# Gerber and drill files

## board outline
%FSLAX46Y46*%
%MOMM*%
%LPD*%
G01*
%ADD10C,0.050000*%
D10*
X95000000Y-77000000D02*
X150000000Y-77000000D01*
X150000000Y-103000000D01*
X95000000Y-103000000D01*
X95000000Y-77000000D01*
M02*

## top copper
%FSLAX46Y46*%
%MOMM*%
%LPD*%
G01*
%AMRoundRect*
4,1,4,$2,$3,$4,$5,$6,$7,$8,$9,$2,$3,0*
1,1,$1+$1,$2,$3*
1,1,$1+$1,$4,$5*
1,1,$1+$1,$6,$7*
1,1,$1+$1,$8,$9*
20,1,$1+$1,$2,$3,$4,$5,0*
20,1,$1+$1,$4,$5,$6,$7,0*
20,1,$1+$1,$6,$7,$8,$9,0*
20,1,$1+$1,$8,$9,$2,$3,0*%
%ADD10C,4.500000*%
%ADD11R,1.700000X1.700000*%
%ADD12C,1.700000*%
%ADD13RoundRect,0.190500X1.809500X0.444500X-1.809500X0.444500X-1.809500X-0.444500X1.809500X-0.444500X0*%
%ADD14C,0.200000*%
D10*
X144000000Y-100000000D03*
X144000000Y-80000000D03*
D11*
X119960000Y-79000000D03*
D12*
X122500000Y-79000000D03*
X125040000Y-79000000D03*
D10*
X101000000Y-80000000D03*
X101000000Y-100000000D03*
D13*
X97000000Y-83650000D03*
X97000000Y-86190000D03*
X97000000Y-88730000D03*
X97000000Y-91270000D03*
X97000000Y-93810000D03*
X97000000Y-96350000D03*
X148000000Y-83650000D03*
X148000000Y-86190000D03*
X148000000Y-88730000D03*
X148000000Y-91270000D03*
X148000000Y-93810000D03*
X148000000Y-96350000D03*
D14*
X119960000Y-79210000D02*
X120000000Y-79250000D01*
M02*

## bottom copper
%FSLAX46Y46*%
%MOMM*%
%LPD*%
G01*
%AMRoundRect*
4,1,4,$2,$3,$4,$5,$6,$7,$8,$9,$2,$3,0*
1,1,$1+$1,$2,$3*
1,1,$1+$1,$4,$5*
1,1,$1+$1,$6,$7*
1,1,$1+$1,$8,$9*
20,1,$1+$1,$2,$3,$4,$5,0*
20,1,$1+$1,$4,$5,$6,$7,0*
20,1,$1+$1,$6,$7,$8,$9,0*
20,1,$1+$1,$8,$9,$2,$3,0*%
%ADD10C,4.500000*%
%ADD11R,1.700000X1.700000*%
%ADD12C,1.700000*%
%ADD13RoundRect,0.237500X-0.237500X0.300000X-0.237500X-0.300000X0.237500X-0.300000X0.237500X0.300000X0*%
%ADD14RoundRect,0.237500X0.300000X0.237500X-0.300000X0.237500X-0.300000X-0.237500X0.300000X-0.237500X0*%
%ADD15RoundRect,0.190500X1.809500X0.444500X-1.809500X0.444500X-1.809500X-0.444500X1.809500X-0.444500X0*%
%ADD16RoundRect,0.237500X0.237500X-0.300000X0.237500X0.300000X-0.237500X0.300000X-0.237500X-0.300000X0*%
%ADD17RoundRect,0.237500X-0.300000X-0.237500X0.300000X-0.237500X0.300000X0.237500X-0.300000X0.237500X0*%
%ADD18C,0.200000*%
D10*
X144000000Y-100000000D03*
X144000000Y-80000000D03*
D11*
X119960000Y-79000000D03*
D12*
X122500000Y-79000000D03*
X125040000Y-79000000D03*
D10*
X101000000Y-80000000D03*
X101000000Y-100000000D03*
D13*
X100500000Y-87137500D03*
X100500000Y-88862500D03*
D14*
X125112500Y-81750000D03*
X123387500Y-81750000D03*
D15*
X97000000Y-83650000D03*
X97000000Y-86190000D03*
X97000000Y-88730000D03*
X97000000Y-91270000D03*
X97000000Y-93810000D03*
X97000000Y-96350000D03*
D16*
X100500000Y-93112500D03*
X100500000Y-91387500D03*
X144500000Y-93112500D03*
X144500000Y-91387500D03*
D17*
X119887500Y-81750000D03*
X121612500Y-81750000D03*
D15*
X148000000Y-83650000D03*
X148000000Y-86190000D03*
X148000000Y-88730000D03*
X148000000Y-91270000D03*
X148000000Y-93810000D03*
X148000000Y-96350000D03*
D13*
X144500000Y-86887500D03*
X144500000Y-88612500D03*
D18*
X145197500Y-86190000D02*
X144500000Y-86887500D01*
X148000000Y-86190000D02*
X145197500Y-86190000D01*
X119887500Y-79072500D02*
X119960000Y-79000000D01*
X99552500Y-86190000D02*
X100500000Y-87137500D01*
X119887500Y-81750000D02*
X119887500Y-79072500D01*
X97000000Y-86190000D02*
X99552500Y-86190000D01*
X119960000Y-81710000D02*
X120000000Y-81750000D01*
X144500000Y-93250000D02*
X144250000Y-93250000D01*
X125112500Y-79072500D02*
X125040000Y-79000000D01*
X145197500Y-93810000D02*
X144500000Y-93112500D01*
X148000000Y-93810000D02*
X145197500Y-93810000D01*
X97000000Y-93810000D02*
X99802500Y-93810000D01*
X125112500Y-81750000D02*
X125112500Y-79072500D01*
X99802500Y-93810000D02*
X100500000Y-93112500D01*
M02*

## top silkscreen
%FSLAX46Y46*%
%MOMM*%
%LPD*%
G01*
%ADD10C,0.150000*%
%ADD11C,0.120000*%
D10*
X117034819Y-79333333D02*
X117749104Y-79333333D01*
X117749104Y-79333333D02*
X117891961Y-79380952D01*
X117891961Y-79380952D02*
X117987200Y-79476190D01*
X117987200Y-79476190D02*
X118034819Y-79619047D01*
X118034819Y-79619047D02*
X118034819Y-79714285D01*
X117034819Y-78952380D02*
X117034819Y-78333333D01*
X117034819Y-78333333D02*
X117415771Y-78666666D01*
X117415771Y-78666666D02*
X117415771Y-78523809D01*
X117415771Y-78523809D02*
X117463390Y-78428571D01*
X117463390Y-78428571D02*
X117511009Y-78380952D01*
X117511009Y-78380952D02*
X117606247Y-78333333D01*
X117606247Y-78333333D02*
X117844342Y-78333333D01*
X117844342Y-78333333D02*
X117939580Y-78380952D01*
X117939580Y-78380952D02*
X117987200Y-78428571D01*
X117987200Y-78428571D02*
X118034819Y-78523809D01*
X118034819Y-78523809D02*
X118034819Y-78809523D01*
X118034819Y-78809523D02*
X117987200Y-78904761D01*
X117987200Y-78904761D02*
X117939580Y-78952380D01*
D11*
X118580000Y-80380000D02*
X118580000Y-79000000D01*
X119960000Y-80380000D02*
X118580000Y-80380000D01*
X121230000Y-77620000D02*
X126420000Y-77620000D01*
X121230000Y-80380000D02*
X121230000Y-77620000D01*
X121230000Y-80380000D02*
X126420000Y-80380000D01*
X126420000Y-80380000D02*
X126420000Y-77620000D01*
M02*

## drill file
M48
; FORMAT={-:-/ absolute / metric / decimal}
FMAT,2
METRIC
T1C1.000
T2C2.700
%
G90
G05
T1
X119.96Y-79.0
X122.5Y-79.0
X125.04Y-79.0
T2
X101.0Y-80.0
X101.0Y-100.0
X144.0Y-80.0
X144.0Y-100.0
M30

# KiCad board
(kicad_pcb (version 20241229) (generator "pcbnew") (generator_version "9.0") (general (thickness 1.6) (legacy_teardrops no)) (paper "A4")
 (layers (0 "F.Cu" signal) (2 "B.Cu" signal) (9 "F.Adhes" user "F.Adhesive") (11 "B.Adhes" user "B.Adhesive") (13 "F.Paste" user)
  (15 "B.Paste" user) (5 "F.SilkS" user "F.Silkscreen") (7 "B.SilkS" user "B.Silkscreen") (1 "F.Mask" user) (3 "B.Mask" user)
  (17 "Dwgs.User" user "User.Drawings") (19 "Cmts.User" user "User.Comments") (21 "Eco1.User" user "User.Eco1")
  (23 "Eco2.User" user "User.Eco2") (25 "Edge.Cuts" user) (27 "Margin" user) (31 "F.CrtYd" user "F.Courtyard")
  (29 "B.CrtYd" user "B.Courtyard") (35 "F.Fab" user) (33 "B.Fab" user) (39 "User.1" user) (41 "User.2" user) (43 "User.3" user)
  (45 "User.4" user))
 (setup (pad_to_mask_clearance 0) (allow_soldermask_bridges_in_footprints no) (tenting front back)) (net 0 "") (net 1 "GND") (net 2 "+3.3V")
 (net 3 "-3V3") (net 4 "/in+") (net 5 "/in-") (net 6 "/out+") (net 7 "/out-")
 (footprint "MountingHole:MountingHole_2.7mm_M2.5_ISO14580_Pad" (layer "F.Cu") (at 144 100)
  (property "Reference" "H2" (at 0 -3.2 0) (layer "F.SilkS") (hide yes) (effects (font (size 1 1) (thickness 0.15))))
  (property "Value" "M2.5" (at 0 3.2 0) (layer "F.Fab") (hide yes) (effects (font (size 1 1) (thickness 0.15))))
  (pad "1" thru_hole circle (at 0 0) (size 4.5 4.5) (drill 2.7) (layers "*.Cu" "*.Mask") (remove_unused_layers no) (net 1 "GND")
   (zone_connect 2)))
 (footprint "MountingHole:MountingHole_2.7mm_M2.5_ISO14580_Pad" (layer "F.Cu") (at 144 80)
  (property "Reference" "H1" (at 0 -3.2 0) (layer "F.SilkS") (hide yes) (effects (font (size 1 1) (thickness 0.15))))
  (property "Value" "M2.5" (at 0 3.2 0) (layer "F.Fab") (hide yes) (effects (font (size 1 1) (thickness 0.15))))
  (pad "1" thru_hole circle (at 0 0) (size 4.5 4.5) (drill 2.7) (layers "*.Cu" "*.Mask") (remove_unused_layers no) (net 1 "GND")
   (zone_connect 2)))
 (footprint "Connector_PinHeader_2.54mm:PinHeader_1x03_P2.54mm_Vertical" (layer "F.Cu") (at 119.96 79 90)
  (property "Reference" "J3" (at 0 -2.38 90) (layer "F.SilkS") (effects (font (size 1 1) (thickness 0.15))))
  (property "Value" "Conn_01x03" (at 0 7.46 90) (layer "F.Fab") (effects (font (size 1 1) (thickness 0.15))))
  (fp_line (start -1.38 -1.38) (end 0 -1.38) (stroke (width 0.12) (type solid)) (layer "F.SilkS"))
  (fp_line (start -1.38 0) (end -1.38 -1.38) (stroke (width 0.12) (type solid)) (layer "F.SilkS"))
  (fp_line (start 1.38 1.27) (end 1.38 6.46) (stroke (width 0.12) (type solid)) (layer "F.SilkS"))
  (fp_line (start -1.38 1.27) (end 1.38 1.27) (stroke (width 0.12) (type solid)) (layer "F.SilkS"))
  (fp_line (start -1.38 1.27) (end -1.38 6.46) (stroke (width 0.12) (type solid)) (layer "F.SilkS"))
  (fp_line (start -1.38 6.46) (end 1.38 6.46) (stroke (width 0.12) (type solid)) (layer "F.SilkS"))
  (pad "1" thru_hole rect (at 0 0 90) (size 1.7 1.7) (drill 1) (layers "*.Cu" "*.Mask") (remove_unused_layers no) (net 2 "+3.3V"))
  (pad "2" thru_hole circle (at 0 2.54 90) (size 1.7 1.7) (drill 1) (layers "*.Cu" "*.Mask") (remove_unused_layers no) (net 1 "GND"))
  (pad "3" thru_hole circle (at 0 5.08 90) (size 1.7 1.7) (drill 1) (layers "*.Cu" "*.Mask") (remove_unused_layers no) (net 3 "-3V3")))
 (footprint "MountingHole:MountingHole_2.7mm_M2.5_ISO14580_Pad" (layer "F.Cu") (at 101 80)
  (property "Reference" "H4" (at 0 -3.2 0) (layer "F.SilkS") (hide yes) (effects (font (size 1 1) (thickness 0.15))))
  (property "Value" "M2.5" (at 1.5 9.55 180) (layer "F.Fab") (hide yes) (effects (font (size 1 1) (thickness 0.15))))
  (pad "1" thru_hole circle (at 0 0) (size 4.5 4.5) (drill 2.7) (layers "*.Cu" "*.Mask") (remove_unused_layers no) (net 1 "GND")
   (zone_connect 2)))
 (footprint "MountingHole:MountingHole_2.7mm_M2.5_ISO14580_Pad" (layer "F.Cu") (at 101 100)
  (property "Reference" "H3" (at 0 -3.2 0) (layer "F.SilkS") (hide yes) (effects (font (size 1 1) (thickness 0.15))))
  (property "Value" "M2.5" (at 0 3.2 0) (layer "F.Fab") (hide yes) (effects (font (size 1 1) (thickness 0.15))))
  (pad "1" thru_hole circle (at 0 0) (size 4.5 4.5) (drill 2.7) (layers "*.Cu" "*.Mask") (remove_unused_layers no) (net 1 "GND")
   (zone_connect 2)))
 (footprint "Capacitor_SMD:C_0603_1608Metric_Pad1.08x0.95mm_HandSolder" (layer "B.Cu") (at 100.5 88 -90)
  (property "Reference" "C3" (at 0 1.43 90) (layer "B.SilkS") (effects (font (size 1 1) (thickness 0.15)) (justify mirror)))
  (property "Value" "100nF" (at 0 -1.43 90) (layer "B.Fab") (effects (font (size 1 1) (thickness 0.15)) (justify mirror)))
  (pad "1" smd roundrect (at -0.8625 0 270) (size 1.075 0.95) (layers "B.Cu" "B.Mask" "B.Paste") (roundrect_rratio 0.25) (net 2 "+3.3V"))
  (pad "2" smd roundrect (at 0.8625 0 270) (size 1.075 0.95) (layers "B.Cu" "B.Mask" "B.Paste") (roundrect_rratio 0.25) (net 1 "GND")))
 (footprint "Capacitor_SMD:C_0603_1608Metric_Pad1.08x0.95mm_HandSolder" (layer "B.Cu") (at 124.25 81.75 180)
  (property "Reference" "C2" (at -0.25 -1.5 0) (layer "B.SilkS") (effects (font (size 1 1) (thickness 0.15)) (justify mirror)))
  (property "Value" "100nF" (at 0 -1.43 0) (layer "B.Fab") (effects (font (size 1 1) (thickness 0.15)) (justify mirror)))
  (pad "1" smd roundrect (at -0.8625 0 180) (size 1.075 0.95) (layers "B.Cu" "B.Mask" "B.Paste") (roundrect_rratio 0.25) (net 3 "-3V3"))
  (pad "2" smd roundrect (at 0.8625 0 180) (size 1.075 0.95) (layers "B.Cu" "B.Mask" "B.Paste") (roundrect_rratio 0.25) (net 1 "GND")))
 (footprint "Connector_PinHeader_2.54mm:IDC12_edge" (layer "B.Cu") (at 97 83.65 180)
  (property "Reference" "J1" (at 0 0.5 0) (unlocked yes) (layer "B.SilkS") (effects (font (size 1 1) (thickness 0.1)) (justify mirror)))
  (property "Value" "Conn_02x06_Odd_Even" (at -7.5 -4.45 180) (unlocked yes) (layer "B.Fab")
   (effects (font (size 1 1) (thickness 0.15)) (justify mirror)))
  (pad "1" smd roundrect (at 0 0 180) (size 4 1.27) (layers "B.Cu" "B.Mask" "B.Paste") (roundrect_rratio 0.15) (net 1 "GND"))
  (pad "2" smd roundrect (at 0 0 180) (size 4 1.27) (layers "F.Cu" "F.Mask" "F.Paste") (roundrect_rratio 0.15) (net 1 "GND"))
  (pad "3" smd roundrect (at 0 -2.54 180) (size 4 1.27) (layers "B.Cu" "B.Mask" "B.Paste") (roundrect_rratio 0.15) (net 2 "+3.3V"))
  (pad "4" smd roundrect (at 0 -2.54 180) (size 4 1.27) (layers "F.Cu" "F.Mask" "F.Paste") (roundrect_rratio 0.15) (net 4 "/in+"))
  (pad "5" smd roundrect (at 0 -5.08 180) (size 4 1.27) (layers "B.Cu" "B.Mask" "B.Paste") (roundrect_rratio 0.15) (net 1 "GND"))
  (pad "6" smd roundrect (at 0 -5.08 180) (size 4 1.27) (layers "F.Cu" "F.Mask" "F.Paste") (roundrect_rratio 0.15) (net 1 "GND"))
  (pad "7" smd roundrect (at 0 -7.62 180) (size 4 1.27) (layers "B.Cu" "B.Mask" "B.Paste") (roundrect_rratio 0.15) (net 1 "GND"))
  (pad "8" smd roundrect (at 0 -7.62 180) (size 4 1.27) (layers "F.Cu" "F.Mask" "F.Paste") (roundrect_rratio 0.15) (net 1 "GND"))
  (pad "9" smd roundrect (at 0 -10.16 180) (size 4 1.27) (layers "B.Cu" "B.Mask" "B.Paste") (roundrect_rratio 0.15) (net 3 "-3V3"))
  (pad "10" smd roundrect (at 0 -10.16 180) (size 4 1.27) (layers "F.Cu" "F.Mask" "F.Paste") (roundrect_rratio 0.15) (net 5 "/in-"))
  (pad "11" smd roundrect (at 0 -12.7 180) (size 4 1.27) (layers "B.Cu" "B.Mask" "B.Paste") (roundrect_rratio 0.15) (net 1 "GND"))
  (pad "12" smd roundrect (at 0 -12.7 180) (size 4 1.27) (layers "F.Cu" "F.Mask" "F.Paste") (roundrect_rratio 0.15) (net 1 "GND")))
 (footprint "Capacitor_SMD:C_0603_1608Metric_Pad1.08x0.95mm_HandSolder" (layer "B.Cu") (at 100.5 92.25 90)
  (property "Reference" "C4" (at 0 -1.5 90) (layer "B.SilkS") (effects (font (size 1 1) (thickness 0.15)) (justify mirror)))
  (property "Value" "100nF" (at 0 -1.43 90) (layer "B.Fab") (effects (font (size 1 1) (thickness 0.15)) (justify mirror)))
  (pad "1" smd roundrect (at -0.8625 0 90) (size 1.075 0.95) (layers "B.Cu" "B.Mask" "B.Paste") (roundrect_rratio 0.25) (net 3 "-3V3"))
  (pad "2" smd roundrect (at 0.8625 0 90) (size 1.075 0.95) (layers "B.Cu" "B.Mask" "B.Paste") (roundrect_rratio 0.25) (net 1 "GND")))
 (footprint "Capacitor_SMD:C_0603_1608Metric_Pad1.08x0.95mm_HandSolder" (layer "B.Cu") (at 144.5 92.25 90)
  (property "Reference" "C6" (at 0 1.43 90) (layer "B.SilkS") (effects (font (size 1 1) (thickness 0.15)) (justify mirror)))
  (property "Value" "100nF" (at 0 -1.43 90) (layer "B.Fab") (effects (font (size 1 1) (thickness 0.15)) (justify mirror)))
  (pad "1" smd roundrect (at -0.8625 0 90) (size 1.075 0.95) (layers "B.Cu" "B.Mask" "B.Paste") (roundrect_rratio 0.25) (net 3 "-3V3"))
  (pad "2" smd roundrect (at 0.8625 0 90) (size 1.075 0.95) (layers "B.Cu" "B.Mask" "B.Paste") (roundrect_rratio 0.25) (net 1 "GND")))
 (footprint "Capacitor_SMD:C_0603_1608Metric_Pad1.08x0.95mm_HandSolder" (layer "B.Cu") (at 120.75 81.75)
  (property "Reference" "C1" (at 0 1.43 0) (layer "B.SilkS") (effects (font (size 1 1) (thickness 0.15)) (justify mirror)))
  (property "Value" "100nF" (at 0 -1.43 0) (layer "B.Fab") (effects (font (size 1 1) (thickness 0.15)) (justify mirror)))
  (pad "1" smd roundrect (at -0.8625 0) (size 1.075 0.95) (layers "B.Cu" "B.Mask" "B.Paste") (roundrect_rratio 0.25) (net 2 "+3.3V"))
  (pad "2" smd roundrect (at 0.8625 0) (size 1.075 0.95) (layers "B.Cu" "B.Mask" "B.Paste") (roundrect_rratio 0.25) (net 1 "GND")))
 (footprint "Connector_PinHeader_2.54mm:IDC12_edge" (layer "B.Cu") (at 148 83.65 180)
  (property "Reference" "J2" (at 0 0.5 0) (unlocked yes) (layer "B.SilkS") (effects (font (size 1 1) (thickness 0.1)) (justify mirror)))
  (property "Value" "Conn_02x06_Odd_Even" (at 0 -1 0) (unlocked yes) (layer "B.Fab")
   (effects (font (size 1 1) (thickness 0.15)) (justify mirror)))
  (pad "1" smd roundrect (at 0 0 180) (size 4 1.27) (layers "B.Cu" "B.Mask" "B.Paste") (roundrect_rratio 0.15) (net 1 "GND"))
  (pad "2" smd roundrect (at 0 0 180) (size 4 1.27) (layers "F.Cu" "F.Mask" "F.Paste") (roundrect_rratio 0.15) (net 1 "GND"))
  (pad "3" smd roundrect (at 0 -2.54 180) (size 4 1.27) (layers "B.Cu" "B.Mask" "B.Paste") (roundrect_rratio 0.15) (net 2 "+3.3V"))
  (pad "4" smd roundrect (at 0 -2.54 180) (size 4 1.27) (layers "F.Cu" "F.Mask" "F.Paste") (roundrect_rratio 0.15) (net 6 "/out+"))
  (pad "5" smd roundrect (at 0 -5.08 180) (size 4 1.27) (layers "B.Cu" "B.Mask" "B.Paste") (roundrect_rratio 0.15) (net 1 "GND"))
  (pad "6" smd roundrect (at 0 -5.08 180) (size 4 1.27) (layers "F.Cu" "F.Mask" "F.Paste") (roundrect_rratio 0.15) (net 1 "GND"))
  (pad "7" smd roundrect (at 0 -7.62 180) (size 4 1.27) (layers "B.Cu" "B.Mask" "B.Paste") (roundrect_rratio 0.15) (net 1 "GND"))
  (pad "8" smd roundrect (at 0 -7.62 180) (size 4 1.27) (layers "F.Cu" "F.Mask" "F.Paste") (roundrect_rratio 0.15) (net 1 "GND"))
  (pad "9" smd roundrect (at 0 -10.16 180) (size 4 1.27) (layers "B.Cu" "B.Mask" "B.Paste") (roundrect_rratio 0.15) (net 3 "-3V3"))
  (pad "10" smd roundrect (at 0 -10.16 180) (size 4 1.27) (layers "F.Cu" "F.Mask" "F.Paste") (roundrect_rratio 0.15) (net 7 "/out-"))
  (pad "11" smd roundrect (at 0 -12.7 180) (size 4 1.27) (layers "B.Cu" "B.Mask" "B.Paste") (roundrect_rratio 0.15) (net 1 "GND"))
  (pad "12" smd roundrect (at 0 -12.7 180) (size 4 1.27) (layers "F.Cu" "F.Mask" "F.Paste") (roundrect_rratio 0.15) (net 1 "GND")))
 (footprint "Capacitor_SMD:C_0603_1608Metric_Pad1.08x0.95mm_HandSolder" (layer "B.Cu") (at 144.5 87.75 -90)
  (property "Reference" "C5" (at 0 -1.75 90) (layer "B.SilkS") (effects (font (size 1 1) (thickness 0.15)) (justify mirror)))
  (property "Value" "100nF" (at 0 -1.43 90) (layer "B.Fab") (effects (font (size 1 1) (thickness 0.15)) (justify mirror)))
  (pad "1" smd roundrect (at -0.8625 0 270) (size 1.075 0.95) (layers "B.Cu" "B.Mask" "B.Paste") (roundrect_rratio 0.25) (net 2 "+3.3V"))
  (pad "2" smd roundrect (at 0.8625 0 270) (size 1.075 0.95) (layers "B.Cu" "B.Mask" "B.Paste") (roundrect_rratio 0.25) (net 1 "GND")))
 (gr_rect (start 95 77) (end 150 103) (stroke (width 0.05) (type default)) (fill no) (layer "Edge.Cuts"))
 (segment (start 119.96 79.21) (end 120 79.25) (width 0.2) (layer "F.Cu") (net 2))
 (segment (start 145.1975 86.19) (end 144.5 86.8875) (width 0.2) (layer "B.Cu") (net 2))
 (segment (start 148 86.19) (end 145.1975 86.19) (width 0.2) (layer "B.Cu") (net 2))
 (segment (start 119.8875 79.0725) (end 119.96 79) (width 0.2) (layer "B.Cu") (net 2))
 (segment (start 99.5525 86.19) (end 100.5 87.1375) (width 0.2) (layer "B.Cu") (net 2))
 (segment (start 119.8875 81.75) (end 119.8875 79.0725) (width 0.2) (layer "B.Cu") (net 2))
 (segment (start 97 86.19) (end 99.5525 86.19) (width 0.2) (layer "B.Cu") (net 2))
 (segment (start 119.96 81.71) (end 120 81.75) (width 0.2) (layer "B.Cu") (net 2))
 (segment (start 144.5 93.25) (end 144.25 93.25) (width 0.2) (layer "B.Cu") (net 3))
 (segment (start 125.1125 79.0725) (end 125.04 79) (width 0.2) (layer "B.Cu") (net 3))
 (segment (start 145.1975 93.81) (end 144.5 93.1125) (width 0.2) (layer "B.Cu") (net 3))
 (segment (start 148 93.81) (end 145.1975 93.81) (width 0.2) (layer "B.Cu") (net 3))
 (segment (start 97 93.81) (end 99.8025 93.81) (width 0.2) (layer "B.Cu") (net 3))
 (segment (start 125.1125 81.75) (end 125.1125 79.0725) (width 0.2) (layer "B.Cu") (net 3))
 (segment (start 99.8025 93.81) (end 100.5 93.1125) (width 0.2) (layer "B.Cu") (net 3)))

